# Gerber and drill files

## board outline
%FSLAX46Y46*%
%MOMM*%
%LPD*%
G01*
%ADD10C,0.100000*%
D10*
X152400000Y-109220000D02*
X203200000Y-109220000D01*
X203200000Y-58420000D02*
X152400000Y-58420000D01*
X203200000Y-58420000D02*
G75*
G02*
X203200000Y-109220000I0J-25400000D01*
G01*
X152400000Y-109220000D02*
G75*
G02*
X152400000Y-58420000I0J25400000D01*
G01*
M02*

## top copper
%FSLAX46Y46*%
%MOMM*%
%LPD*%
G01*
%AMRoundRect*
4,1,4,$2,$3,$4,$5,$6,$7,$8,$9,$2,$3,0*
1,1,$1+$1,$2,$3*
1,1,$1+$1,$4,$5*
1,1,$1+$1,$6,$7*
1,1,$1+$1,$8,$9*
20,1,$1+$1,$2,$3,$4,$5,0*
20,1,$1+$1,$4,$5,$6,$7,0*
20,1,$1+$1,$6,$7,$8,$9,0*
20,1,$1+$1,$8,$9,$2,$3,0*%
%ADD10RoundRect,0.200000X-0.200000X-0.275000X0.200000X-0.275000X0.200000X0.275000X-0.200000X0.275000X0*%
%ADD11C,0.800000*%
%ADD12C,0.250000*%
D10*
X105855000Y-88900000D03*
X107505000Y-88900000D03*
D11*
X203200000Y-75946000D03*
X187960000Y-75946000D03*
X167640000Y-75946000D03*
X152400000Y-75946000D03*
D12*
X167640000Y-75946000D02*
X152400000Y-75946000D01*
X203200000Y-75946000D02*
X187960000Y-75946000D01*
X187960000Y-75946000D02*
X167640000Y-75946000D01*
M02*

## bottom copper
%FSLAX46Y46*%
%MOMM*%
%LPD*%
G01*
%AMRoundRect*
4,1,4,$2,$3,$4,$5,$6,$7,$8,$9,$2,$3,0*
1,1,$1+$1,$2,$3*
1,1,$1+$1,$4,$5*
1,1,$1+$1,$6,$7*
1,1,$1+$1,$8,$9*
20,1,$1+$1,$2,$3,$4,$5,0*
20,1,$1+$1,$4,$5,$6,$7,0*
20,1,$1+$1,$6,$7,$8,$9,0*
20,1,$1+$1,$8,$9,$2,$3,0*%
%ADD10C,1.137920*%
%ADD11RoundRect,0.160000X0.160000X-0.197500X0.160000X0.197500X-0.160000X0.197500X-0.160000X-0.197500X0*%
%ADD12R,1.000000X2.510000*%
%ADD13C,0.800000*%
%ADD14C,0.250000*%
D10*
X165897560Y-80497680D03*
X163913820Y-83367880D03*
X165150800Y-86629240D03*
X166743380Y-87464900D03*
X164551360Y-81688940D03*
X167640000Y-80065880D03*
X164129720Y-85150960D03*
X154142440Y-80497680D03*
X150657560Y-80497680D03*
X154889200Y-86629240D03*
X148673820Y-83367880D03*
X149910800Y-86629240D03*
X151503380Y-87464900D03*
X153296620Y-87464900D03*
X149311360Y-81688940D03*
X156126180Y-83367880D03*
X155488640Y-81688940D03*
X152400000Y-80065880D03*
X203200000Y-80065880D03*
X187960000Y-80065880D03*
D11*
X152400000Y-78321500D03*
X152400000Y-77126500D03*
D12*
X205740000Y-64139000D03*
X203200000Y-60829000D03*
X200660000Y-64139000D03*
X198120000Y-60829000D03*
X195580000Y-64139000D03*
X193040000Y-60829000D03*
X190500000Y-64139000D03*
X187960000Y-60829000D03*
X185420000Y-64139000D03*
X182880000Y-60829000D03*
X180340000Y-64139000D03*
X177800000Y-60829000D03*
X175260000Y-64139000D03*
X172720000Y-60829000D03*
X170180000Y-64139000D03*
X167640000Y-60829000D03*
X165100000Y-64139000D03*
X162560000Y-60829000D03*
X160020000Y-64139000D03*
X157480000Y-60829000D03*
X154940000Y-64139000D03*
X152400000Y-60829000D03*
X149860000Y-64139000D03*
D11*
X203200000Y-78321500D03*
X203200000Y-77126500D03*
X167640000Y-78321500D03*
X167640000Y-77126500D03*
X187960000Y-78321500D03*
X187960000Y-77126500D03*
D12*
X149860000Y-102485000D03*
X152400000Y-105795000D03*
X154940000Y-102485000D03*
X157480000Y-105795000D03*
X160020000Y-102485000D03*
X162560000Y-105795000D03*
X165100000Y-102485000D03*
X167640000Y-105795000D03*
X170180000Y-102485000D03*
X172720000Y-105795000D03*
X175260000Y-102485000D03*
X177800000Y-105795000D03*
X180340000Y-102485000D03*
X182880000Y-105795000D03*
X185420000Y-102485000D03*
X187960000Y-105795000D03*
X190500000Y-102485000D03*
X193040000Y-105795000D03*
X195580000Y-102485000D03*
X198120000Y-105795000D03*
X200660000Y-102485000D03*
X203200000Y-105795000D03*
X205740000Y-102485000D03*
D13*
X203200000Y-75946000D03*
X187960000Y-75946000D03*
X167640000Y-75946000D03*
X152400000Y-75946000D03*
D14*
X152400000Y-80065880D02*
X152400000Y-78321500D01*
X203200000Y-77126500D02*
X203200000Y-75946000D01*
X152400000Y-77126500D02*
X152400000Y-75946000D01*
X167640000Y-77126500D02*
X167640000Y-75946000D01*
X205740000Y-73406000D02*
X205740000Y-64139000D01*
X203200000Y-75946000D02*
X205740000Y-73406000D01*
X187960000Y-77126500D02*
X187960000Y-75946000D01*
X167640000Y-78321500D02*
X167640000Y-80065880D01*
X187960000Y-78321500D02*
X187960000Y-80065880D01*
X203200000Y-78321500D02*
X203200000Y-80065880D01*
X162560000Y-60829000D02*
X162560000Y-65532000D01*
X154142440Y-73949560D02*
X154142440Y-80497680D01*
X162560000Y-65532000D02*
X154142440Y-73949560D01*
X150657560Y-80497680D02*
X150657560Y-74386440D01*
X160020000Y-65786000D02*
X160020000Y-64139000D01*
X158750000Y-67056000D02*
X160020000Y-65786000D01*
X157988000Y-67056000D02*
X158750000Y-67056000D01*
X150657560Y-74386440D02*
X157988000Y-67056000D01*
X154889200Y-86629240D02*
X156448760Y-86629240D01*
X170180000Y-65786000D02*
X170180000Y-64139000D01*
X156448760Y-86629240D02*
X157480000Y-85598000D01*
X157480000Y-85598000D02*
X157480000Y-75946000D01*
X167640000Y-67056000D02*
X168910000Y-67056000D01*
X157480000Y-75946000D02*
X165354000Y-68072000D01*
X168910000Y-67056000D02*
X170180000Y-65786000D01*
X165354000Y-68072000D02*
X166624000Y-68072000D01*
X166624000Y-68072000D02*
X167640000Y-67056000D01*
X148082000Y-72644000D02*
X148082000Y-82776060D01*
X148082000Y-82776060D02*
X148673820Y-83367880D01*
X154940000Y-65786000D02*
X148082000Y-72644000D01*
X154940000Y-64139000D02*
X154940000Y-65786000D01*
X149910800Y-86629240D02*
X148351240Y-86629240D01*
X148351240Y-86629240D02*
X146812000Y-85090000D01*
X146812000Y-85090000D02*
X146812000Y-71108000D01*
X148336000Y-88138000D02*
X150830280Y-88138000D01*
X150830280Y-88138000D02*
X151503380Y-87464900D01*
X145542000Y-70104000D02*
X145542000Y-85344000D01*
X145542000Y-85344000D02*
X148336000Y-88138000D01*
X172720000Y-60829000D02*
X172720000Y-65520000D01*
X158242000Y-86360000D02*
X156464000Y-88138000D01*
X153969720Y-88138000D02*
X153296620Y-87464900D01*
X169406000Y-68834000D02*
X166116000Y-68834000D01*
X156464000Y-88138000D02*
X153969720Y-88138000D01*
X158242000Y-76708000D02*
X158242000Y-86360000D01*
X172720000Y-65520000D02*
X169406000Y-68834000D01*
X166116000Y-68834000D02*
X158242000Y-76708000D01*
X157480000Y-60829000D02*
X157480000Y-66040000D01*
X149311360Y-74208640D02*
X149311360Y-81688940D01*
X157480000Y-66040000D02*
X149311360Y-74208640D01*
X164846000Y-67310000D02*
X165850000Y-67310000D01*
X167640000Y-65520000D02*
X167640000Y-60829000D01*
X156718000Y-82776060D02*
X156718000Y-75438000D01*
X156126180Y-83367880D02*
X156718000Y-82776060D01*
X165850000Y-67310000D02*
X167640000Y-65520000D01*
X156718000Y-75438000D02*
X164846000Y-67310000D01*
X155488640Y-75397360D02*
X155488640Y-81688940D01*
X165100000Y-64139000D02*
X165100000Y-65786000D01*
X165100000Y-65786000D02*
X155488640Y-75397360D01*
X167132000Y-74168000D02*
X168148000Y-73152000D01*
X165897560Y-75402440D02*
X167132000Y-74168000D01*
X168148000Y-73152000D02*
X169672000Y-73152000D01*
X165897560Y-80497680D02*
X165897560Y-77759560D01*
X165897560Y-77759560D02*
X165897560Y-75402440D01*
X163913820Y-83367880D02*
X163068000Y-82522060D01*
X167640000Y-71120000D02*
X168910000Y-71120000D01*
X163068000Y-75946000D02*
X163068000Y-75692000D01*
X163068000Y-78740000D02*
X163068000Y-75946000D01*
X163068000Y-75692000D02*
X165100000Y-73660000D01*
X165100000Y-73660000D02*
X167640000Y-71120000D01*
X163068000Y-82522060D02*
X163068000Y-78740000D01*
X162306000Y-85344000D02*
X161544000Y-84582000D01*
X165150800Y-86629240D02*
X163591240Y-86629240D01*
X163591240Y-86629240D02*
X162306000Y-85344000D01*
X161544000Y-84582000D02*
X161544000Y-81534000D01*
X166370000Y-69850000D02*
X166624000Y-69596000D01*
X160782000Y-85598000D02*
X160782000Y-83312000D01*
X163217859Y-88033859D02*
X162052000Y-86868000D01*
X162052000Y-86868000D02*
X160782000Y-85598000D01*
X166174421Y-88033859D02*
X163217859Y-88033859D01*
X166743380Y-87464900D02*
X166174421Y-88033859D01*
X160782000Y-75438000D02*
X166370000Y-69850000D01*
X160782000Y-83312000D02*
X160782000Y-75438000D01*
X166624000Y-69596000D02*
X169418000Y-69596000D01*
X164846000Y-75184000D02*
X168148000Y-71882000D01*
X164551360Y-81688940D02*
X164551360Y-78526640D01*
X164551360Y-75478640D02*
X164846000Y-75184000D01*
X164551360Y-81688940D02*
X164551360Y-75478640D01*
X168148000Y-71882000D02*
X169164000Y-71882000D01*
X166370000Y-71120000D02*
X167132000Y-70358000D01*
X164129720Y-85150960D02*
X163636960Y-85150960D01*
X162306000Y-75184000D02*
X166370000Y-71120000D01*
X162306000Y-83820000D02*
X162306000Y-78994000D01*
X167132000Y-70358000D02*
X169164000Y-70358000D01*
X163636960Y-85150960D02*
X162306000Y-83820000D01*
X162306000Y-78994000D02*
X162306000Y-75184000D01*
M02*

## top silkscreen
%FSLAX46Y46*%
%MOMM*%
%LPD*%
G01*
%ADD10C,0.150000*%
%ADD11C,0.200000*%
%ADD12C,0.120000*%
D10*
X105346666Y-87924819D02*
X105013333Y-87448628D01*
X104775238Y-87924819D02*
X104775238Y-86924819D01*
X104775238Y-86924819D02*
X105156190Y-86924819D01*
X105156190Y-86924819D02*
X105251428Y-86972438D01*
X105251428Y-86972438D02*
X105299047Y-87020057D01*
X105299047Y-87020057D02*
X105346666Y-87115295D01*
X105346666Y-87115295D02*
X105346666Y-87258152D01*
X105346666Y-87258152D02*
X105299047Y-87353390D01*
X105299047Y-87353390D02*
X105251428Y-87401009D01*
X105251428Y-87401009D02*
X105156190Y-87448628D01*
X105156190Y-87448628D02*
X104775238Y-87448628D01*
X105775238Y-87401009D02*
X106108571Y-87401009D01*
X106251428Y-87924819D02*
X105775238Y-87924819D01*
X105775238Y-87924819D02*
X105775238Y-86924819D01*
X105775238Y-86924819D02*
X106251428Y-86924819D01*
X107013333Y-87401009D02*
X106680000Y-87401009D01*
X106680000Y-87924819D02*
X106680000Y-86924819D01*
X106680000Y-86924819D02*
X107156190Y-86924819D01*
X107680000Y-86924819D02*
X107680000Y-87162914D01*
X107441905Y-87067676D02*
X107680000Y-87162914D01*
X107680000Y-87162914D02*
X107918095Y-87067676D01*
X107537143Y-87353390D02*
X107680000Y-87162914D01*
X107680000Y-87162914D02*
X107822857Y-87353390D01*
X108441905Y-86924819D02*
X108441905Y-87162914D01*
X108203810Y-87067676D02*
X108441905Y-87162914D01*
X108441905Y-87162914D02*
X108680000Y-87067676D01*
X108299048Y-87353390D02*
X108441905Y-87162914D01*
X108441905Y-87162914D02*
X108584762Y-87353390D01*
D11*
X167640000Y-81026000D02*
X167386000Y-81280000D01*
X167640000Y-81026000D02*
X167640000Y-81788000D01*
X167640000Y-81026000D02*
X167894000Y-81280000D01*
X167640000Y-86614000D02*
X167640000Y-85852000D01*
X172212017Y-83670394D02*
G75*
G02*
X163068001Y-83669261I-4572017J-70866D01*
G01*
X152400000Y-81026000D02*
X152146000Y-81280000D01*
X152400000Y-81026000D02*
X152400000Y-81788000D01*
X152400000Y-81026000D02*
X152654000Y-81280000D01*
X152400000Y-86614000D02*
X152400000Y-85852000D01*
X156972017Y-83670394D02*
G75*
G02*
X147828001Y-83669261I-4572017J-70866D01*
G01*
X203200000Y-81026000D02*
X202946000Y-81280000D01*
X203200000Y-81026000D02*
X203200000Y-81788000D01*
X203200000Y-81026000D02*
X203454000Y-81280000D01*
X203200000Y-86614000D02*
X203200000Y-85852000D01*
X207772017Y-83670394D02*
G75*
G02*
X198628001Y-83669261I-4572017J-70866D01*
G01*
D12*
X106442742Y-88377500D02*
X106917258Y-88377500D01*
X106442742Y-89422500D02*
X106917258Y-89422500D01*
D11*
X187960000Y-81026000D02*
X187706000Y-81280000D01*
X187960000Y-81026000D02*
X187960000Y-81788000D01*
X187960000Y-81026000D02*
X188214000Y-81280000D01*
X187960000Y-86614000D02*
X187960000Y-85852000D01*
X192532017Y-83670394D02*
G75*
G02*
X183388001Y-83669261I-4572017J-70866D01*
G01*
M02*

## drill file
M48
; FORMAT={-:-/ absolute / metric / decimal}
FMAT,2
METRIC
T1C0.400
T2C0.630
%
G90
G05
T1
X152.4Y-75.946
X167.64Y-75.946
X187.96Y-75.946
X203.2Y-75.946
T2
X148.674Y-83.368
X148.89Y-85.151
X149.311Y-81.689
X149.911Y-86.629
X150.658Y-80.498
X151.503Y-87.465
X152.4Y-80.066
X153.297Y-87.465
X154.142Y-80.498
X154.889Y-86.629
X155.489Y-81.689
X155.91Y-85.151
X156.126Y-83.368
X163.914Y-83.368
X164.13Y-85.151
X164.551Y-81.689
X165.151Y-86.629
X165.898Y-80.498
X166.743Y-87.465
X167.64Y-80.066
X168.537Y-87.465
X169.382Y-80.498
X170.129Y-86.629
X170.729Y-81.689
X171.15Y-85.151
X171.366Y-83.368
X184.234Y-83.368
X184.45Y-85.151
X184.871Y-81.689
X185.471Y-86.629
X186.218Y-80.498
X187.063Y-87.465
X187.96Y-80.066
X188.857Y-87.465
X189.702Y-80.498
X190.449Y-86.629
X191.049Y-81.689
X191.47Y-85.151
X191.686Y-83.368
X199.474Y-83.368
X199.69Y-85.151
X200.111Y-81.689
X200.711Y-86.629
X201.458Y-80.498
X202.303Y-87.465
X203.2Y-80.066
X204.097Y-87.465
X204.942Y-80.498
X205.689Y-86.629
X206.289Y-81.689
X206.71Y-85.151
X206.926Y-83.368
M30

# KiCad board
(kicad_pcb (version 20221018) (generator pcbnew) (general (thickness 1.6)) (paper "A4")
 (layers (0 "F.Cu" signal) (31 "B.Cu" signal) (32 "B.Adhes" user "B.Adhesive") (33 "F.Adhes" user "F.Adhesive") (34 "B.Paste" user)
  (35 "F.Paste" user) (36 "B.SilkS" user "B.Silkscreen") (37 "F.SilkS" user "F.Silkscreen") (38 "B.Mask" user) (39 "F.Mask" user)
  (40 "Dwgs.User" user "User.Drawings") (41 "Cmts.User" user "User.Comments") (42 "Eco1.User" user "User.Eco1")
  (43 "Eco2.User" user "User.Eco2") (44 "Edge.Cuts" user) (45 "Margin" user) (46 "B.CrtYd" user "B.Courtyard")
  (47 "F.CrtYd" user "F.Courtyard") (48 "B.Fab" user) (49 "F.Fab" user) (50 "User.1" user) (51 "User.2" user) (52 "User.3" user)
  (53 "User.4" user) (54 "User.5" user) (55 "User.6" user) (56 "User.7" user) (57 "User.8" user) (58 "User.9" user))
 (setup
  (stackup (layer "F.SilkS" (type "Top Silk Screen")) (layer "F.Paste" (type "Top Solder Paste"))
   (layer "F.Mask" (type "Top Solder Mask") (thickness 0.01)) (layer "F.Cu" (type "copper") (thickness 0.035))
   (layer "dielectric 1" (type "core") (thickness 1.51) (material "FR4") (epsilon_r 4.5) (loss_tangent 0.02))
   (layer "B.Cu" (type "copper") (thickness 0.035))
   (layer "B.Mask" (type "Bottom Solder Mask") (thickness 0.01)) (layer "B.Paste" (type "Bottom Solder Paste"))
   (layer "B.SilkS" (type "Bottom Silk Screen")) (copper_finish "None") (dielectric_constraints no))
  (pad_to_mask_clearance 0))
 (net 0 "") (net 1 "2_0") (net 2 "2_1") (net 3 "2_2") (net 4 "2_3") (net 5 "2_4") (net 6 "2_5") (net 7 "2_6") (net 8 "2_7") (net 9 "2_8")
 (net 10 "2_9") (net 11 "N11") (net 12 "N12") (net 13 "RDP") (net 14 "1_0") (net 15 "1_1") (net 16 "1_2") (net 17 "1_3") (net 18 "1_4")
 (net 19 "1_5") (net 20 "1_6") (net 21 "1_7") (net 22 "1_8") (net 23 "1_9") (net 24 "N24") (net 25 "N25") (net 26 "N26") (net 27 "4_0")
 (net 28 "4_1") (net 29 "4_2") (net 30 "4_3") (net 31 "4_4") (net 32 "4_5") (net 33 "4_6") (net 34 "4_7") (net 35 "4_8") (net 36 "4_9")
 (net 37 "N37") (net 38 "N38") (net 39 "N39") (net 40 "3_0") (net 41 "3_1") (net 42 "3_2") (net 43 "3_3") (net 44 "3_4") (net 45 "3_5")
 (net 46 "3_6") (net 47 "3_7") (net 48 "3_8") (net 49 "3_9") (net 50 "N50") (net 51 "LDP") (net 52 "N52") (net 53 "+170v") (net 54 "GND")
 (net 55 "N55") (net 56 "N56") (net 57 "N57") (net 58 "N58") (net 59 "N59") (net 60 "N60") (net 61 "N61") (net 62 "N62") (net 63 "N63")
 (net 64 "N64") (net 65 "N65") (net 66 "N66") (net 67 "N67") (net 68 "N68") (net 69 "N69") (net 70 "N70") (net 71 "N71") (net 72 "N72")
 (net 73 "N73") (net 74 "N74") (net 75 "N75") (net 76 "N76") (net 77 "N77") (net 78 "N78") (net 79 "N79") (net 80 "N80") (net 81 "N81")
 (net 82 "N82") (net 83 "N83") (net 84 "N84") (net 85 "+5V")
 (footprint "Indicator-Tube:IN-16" (layer "F.Cu") (at 167.64 83.82)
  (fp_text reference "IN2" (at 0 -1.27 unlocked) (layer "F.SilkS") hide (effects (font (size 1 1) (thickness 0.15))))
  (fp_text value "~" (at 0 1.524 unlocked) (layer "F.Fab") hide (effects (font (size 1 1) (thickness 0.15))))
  (fp_line (start 0 -2.794) (end -0.254 -2.54) (stroke (width 0.2) (type solid)) (layer "F.SilkS"))
  (fp_line (start 0 -2.794) (end 0 -2.032) (stroke (width 0.2) (type solid)) (layer "F.SilkS"))
  (fp_line (start 0 -2.794) (end 0.254 -2.54) (stroke (width 0.2) (type solid)) (layer "F.SilkS"))
  (fp_line (start 0 2.794) (end 0 2.032) (stroke (width 0.2) (type solid)) (layer "F.SilkS"))
  (fp_arc (start 4.572017 -0.149606) (mid -0.000567 4.493826) (end -4.571999 -0.150739) (stroke (width 0.2) (type solid)) (layer "F.SilkS"))
  (pad "0" thru_hole circle (at 1.74244 -3.32232 180) (size 1.13792 1.13792) (drill 0.62992) (layers "*.Cu" "*.Mask") (remove_unused_layers)
   (zone_layer_connections) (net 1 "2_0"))
  (pad "1" thru_hole circle (at -1.74244 -3.32232 180) (size 1.13792 1.13792) (drill 0.62992) (layers "*.Cu" "*.Mask")
   (remove_unused_layers) (zone_layer_connections) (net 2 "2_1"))
  (pad "2" thru_hole circle (at 2.4892 2.80924 180) (size 1.13792 1.13792) (drill 0.62992) (layers "*.Cu" "*.Mask") (remove_unused_layers)
   (zone_layer_connections) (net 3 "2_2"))
  (pad "3" thru_hole circle (at -3.72618 -0.45212 180) (size 1.13792 1.13792) (drill 0.62992) (layers "*.Cu" "*.Mask")
   (remove_unused_layers) (zone_layer_connections) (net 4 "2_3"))
  (pad "4" thru_hole circle (at -2.4892 2.80924 180) (size 1.13792 1.13792) (drill 0.62992) (layers "*.Cu" "*.Mask") (remove_unused_layers)
   (zone_layer_connections) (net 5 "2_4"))
  (pad "5" thru_hole circle (at -0.89662 3.6449 180) (size 1.13792 1.13792) (drill 0.62992) (layers "*.Cu" "*.Mask") (remove_unused_layers)
   (zone_layer_connections) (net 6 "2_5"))
  (pad "6" thru_hole circle (at 0.89662 3.6449 180) (size 1.13792 1.13792) (drill 0.62992) (layers "*.Cu" "*.Mask") (remove_unused_layers)
   (zone_layer_connections) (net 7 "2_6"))
  (pad "7" thru_hole circle (at -3.08864 -2.13106 180) (size 1.13792 1.13792) (drill 0.62992) (layers "*.Cu" "*.Mask")
   (remove_unused_layers) (zone_layer_connections) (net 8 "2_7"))
  (pad "8" thru_hole circle (at 3.72618 -0.45212 180) (size 1.13792 1.13792) (drill 0.62992) (layers "*.Cu" "*.Mask") (remove_unused_layers)
   (zone_layer_connections) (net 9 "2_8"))
  (pad "9" thru_hole circle (at 3.08864 -2.13106 180) (size 1.13792 1.13792) (drill 0.62992) (layers "*.Cu" "*.Mask") (remove_unused_layers)
   (zone_layer_connections) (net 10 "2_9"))
  (pad "A" thru_hole circle (at 0 -3.75412 180) (size 1.13792 1.13792) (drill 0.62992) (layers "*.Cu" "*.Mask") (remove_unused_layers)
   (zone_layer_connections) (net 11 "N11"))
  (pad "LHDP" thru_hole circle (at 3.51028 1.33096 180) (size 1.13792 1.13792) (drill 0.62992) (layers "*.Cu" "*.Mask")
   (remove_unused_layers) (zone_layer_connections) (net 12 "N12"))
  (pad "RHDP" thru_hole circle (at -3.51028 1.33096 180) (size 1.13792 1.13792) (drill 0.62992) (layers "*.Cu" "*.Mask")
   (remove_unused_layers) (zone_layer_connections) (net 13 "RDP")))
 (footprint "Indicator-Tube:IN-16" (layer "F.Cu") (at 152.4 83.82)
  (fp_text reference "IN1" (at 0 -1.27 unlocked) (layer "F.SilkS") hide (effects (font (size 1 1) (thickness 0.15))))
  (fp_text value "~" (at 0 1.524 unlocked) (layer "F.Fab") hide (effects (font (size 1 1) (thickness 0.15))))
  (fp_line (start 0 -2.794) (end -0.254 -2.54) (stroke (width 0.2) (type solid)) (layer "F.SilkS"))
  (fp_line (start 0 -2.794) (end 0 -2.032) (stroke (width 0.2) (type solid)) (layer "F.SilkS"))
  (fp_line (start 0 -2.794) (end 0.254 -2.54) (stroke (width 0.2) (type solid)) (layer "F.SilkS"))
  (fp_line (start 0 2.794) (end 0 2.032) (stroke (width 0.2) (type solid)) (layer "F.SilkS"))
  (fp_arc (start 4.572017 -0.149606) (mid -0.000567 4.493826) (end -4.571999 -0.150739) (stroke (width 0.2) (type solid)) (layer "F.SilkS"))
  (pad "0" thru_hole circle (at 1.74244 -3.32232 180) (size 1.13792 1.13792) (drill 0.62992) (layers "*.Cu" "*.Mask") (remove_unused_layers)
   (zone_layer_connections) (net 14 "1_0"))
  (pad "1" thru_hole circle (at -1.74244 -3.32232 180) (size 1.13792 1.13792) (drill 0.62992) (layers "*.Cu" "*.Mask")
   (remove_unused_layers) (zone_layer_connections) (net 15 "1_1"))
  (pad "2" thru_hole circle (at 2.4892 2.80924 180) (size 1.13792 1.13792) (drill 0.62992) (layers "*.Cu" "*.Mask") (remove_unused_layers)
   (zone_layer_connections) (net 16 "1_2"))
  (pad "3" thru_hole circle (at -3.72618 -0.45212 180) (size 1.13792 1.13792) (drill 0.62992) (layers "*.Cu" "*.Mask")
   (remove_unused_layers) (zone_layer_connections) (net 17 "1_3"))
  (pad "4" thru_hole circle (at -2.4892 2.80924 180) (size 1.13792 1.13792) (drill 0.62992) (layers "*.Cu" "*.Mask") (remove_unused_layers)
   (zone_layer_connections) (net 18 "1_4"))
  (pad "5" thru_hole circle (at -0.89662 3.6449 180) (size 1.13792 1.13792) (drill 0.62992) (layers "*.Cu" "*.Mask") (remove_unused_layers)
   (zone_layer_connections) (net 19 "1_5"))
  (pad "6" thru_hole circle (at 0.89662 3.6449 180) (size 1.13792 1.13792) (drill 0.62992) (layers "*.Cu" "*.Mask") (remove_unused_layers)
   (zone_layer_connections) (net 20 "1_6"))
  (pad "7" thru_hole circle (at -3.08864 -2.13106 180) (size 1.13792 1.13792) (drill 0.62992) (layers "*.Cu" "*.Mask")
   (remove_unused_layers) (zone_layer_connections) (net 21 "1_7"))
  (pad "8" thru_hole circle (at 3.72618 -0.45212 180) (size 1.13792 1.13792) (drill 0.62992) (layers "*.Cu" "*.Mask") (remove_unused_layers)
   (zone_layer_connections) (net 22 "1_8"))
  (pad "9" thru_hole circle (at 3.08864 -2.13106 180) (size 1.13792 1.13792) (drill 0.62992) (layers "*.Cu" "*.Mask") (remove_unused_layers)
   (zone_layer_connections) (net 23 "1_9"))
  (pad "A" thru_hole circle (at 0 -3.75412 180) (size 1.13792 1.13792) (drill 0.62992) (layers "*.Cu" "*.Mask") (remove_unused_layers)
   (zone_layer_connections) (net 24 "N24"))
  (pad "LHDP" thru_hole circle (at 3.51028 1.33096 180) (size 1.13792 1.13792) (drill 0.62992) (layers "*.Cu" "*.Mask")
   (remove_unused_layers) (zone_layer_connections) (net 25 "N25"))
  (pad "RHDP" thru_hole circle (at -3.51028 1.33096 180) (size 1.13792 1.13792) (drill 0.62992) (layers "*.Cu" "*.Mask")
   (remove_unused_layers) (zone_layer_connections) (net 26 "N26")))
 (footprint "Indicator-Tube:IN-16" (layer "F.Cu") (at 203.2 83.82)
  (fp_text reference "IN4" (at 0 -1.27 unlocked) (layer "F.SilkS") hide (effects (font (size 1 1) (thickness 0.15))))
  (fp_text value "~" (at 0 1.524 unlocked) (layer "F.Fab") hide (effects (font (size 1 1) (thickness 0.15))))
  (fp_line (start 0 -2.794) (end -0.254 -2.54) (stroke (width 0.2) (type solid)) (layer "F.SilkS"))
  (fp_line (start 0 -2.794) (end 0 -2.032) (stroke (width 0.2) (type solid)) (layer "F.SilkS"))
  (fp_line (start 0 -2.794) (end 0.254 -2.54) (stroke (width 0.2) (type solid)) (layer "F.SilkS"))
  (fp_line (start 0 2.794) (end 0 2.032) (stroke (width 0.2) (type solid)) (layer "F.SilkS"))
  (fp_arc (start 4.572017 -0.149606) (mid -0.000567 4.493826) (end -4.571999 -0.150739) (stroke (width 0.2) (type solid)) (layer "F.SilkS"))
  (pad "0" thru_hole circle (at 1.74244 -3.32232 180) (size 1.13792 1.13792) (drill 0.62992) (layers "*.Cu" "*.Mask") (remove_unused_layers)
   (zone_layer_connections) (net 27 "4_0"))
  (pad "1" thru_hole circle (at -1.74244 -3.32232 180) (size 1.13792 1.13792) (drill 0.62992) (layers "*.Cu" "*.Mask")
   (remove_unused_layers) (zone_layer_connections) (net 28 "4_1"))
  (pad "2" thru_hole circle (at 2.4892 2.80924 180) (size 1.13792 1.13792) (drill 0.62992) (layers "*.Cu" "*.Mask") (remove_unused_layers)
   (zone_layer_connections) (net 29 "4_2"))
  (pad "3" thru_hole circle (at -3.72618 -0.45212 180) (size 1.13792 1.13792) (drill 0.62992) (layers "*.Cu" "*.Mask")
   (remove_unused_layers) (zone_layer_connections) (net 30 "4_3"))
  (pad "4" thru_hole circle (at -2.4892 2.80924 180) (size 1.13792 1.13792) (drill 0.62992) (layers "*.Cu" "*.Mask") (remove_unused_layers)
   (zone_layer_connections) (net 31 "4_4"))
  (pad "5" thru_hole circle (at -0.89662 3.6449 180) (size 1.13792 1.13792) (drill 0.62992) (layers "*.Cu" "*.Mask") (remove_unused_layers)
   (zone_layer_connections) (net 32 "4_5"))
  (pad "6" thru_hole circle (at 0.89662 3.6449 180) (size 1.13792 1.13792) (drill 0.62992) (layers "*.Cu" "*.Mask") (remove_unused_layers)
   (zone_layer_connections) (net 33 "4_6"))
  (pad "7" thru_hole circle (at -3.08864 -2.13106 180) (size 1.13792 1.13792) (drill 0.62992) (layers "*.Cu" "*.Mask")
   (remove_unused_layers) (zone_layer_connections) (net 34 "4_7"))
  (pad "8" thru_hole circle (at 3.72618 -0.45212 180) (size 1.13792 1.13792) (drill 0.62992) (layers "*.Cu" "*.Mask") (remove_unused_layers)
   (zone_layer_connections) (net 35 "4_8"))
  (pad "9" thru_hole circle (at 3.08864 -2.13106 180) (size 1.13792 1.13792) (drill 0.62992) (layers "*.Cu" "*.Mask") (remove_unused_layers)
   (zone_layer_connections) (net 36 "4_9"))
  (pad "A" thru_hole circle (at 0 -3.75412 180) (size 1.13792 1.13792) (drill 0.62992) (layers "*.Cu" "*.Mask") (remove_unused_layers)
   (zone_layer_connections) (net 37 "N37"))
  (pad "LHDP" thru_hole circle (at 3.51028 1.33096 180) (size 1.13792 1.13792) (drill 0.62992) (layers "*.Cu" "*.Mask")
   (remove_unused_layers) (zone_layer_connections) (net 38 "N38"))
  (pad "RHDP" thru_hole circle (at -3.51028 1.33096 180) (size 1.13792 1.13792) (drill 0.62992) (layers "*.Cu" "*.Mask")
   (remove_unused_layers) (zone_layer_connections) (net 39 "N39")))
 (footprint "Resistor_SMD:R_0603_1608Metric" (layer "F.Cu") (at 106.68 88.9)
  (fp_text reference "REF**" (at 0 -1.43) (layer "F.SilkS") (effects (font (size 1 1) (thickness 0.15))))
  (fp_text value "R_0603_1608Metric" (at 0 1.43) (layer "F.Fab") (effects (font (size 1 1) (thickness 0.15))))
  (fp_line (start -0.237258 -0.5225) (end 0.237258 -0.5225) (stroke (width 0.12) (type solid)) (layer "F.SilkS"))
  (fp_line (start -0.237258 0.5225) (end 0.237258 0.5225) (stroke (width 0.12) (type solid)) (layer "F.SilkS"))
  (pad "1" smd roundrect (at -0.825 0) (size 0.8 0.95) (layers "F.Cu" "F.Paste" "F.Mask") (roundrect_rratio 0.25))
  (pad "2" smd roundrect (at 0.825 0) (size 0.8 0.95) (layers "F.Cu" "F.Paste" "F.Mask") (roundrect_rratio 0.25)))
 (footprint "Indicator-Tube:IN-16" (layer "F.Cu") (at 187.96 83.82)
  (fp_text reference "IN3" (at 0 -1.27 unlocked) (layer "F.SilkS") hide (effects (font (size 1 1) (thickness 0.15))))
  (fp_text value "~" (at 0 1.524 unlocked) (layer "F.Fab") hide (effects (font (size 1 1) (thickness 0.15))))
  (fp_line (start 0 -2.794) (end -0.254 -2.54) (stroke (width 0.2) (type solid)) (layer "F.SilkS"))
  (fp_line (start 0 -2.794) (end 0 -2.032) (stroke (width 0.2) (type solid)) (layer "F.SilkS"))
  (fp_line (start 0 -2.794) (end 0.254 -2.54) (stroke (width 0.2) (type solid)) (layer "F.SilkS"))
  (fp_line (start 0 2.794) (end 0 2.032) (stroke (width 0.2) (type solid)) (layer "F.SilkS"))
  (fp_arc (start 4.572017 -0.149606) (mid -0.000567 4.493826) (end -4.571999 -0.150739) (stroke (width 0.2) (type solid)) (layer "F.SilkS"))
  (pad "0" thru_hole circle (at 1.74244 -3.32232 180) (size 1.13792 1.13792) (drill 0.62992) (layers "*.Cu" "*.Mask") (remove_unused_layers)
   (zone_layer_connections) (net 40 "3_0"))
  (pad "1" thru_hole circle (at -1.74244 -3.32232 180) (size 1.13792 1.13792) (drill 0.62992) (layers "*.Cu" "*.Mask")
   (remove_unused_layers) (zone_layer_connections) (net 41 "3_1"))
  (pad "2" thru_hole circle (at 2.4892 2.80924 180) (size 1.13792 1.13792) (drill 0.62992) (layers "*.Cu" "*.Mask") (remove_unused_layers)
   (zone_layer_connections) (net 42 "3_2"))
  (pad "3" thru_hole circle (at -3.72618 -0.45212 180) (size 1.13792 1.13792) (drill 0.62992) (layers "*.Cu" "*.Mask")
   (remove_unused_layers) (zone_layer_connections) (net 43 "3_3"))
  (pad "4" thru_hole circle (at -2.4892 2.80924 180) (size 1.13792 1.13792) (drill 0.62992) (layers "*.Cu" "*.Mask") (remove_unused_layers)
   (zone_layer_connections) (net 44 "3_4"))
  (pad "5" thru_hole circle (at -0.89662 3.6449 180) (size 1.13792 1.13792) (drill 0.62992) (layers "*.Cu" "*.Mask") (remove_unused_layers)
   (zone_layer_connections) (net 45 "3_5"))
  (pad "6" thru_hole circle (at 0.89662 3.6449 180) (size 1.13792 1.13792) (drill 0.62992) (layers "*.Cu" "*.Mask") (remove_unused_layers)
   (zone_layer_connections) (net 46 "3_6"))
  (pad "7" thru_hole circle (at -3.08864 -2.13106 180) (size 1.13792 1.13792) (drill 0.62992) (layers "*.Cu" "*.Mask")
   (remove_unused_layers) (zone_layer_connections) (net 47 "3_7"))
  (pad "8" thru_hole circle (at 3.72618 -0.45212 180) (size 1.13792 1.13792) (drill 0.62992) (layers "*.Cu" "*.Mask") (remove_unused_layers)
   (zone_layer_connections) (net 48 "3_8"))
  (pad "9" thru_hole circle (at 3.08864 -2.13106 180) (size 1.13792 1.13792) (drill 0.62992) (layers "*.Cu" "*.Mask") (remove_unused_layers)
   (zone_layer_connections) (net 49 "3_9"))
  (pad "A" thru_hole circle (at 0 -3.75412 180) (size 1.13792 1.13792) (drill 0.62992) (layers "*.Cu" "*.Mask") (remove_unused_layers)
   (zone_layer_connections) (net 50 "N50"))
  (pad "LHDP" thru_hole circle (at 3.51028 1.33096 180) (size 1.13792 1.13792) (drill 0.62992) (layers "*.Cu" "*.Mask")
   (remove_unused_layers) (zone_layer_connections) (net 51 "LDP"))
  (pad "RHDP" thru_hole circle (at -3.51028 1.33096 180) (size 1.13792 1.13792) (drill 0.62992) (layers "*.Cu" "*.Mask")
   (remove_unused_layers) (zone_layer_connections) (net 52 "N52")))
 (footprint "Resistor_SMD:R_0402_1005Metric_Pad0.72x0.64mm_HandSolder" (layer "B.Cu") (at 152.4 77.724 90)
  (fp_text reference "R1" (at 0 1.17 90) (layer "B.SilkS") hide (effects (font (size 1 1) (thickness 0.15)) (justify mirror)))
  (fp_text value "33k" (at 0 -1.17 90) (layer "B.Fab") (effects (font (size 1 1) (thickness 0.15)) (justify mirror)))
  (pad "1" smd roundrect (at -0.5975 0 90) (size 0.715 0.64) (layers "B.Cu" "B.Paste" "B.Mask") (roundrect_rratio 0.25) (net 24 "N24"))
  (pad "2" smd roundrect (at 0.5975 0 90) (size 0.715 0.64) (layers "B.Cu" "B.Paste" "B.Mask") (roundrect_rratio 0.25) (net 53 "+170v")))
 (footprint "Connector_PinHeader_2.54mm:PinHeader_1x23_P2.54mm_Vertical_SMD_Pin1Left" (layer "B.Cu") (at 177.8 62.484 90)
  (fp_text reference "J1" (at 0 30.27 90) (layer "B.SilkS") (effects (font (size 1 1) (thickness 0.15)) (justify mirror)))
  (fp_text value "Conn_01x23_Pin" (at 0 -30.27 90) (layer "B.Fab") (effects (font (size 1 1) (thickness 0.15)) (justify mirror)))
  (pad "1" smd rect (at -1.655 27.94 90) (size 2.51 1) (layers "B.Cu" "B.Paste" "B.Mask") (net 53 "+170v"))
  (pad "2" smd rect (at 1.655 25.4 90) (size 2.51 1) (layers "B.Cu" "B.Paste" "B.Mask") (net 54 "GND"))
  (pad "3" smd rect (at -1.655 22.86 90) (size 2.51 1) (layers "B.Cu" "B.Paste" "B.Mask") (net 13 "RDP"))
  (pad "4" smd rect (at 1.655 20.32 90) (size 2.51 1) (layers "B.Cu" "B.Paste" "B.Mask") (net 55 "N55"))
  (pad "5" smd rect (at -1.655 17.78 90) (size 2.51 1) (layers "B.Cu" "B.Paste" "B.Mask") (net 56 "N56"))
  (pad "6" smd rect (at 1.655 15.24 90) (size 2.51 1) (layers "B.Cu" "B.Paste" "B.Mask") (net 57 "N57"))
  (pad "7" smd rect (at -1.655 12.7 90) (size 2.51 1) (layers "B.Cu" "B.Paste" "B.Mask") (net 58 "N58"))
  (pad "8" smd rect (at 1.655 10.16 90) (size 2.51 1) (layers "B.Cu" "B.Paste" "B.Mask") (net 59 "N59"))
  (pad "9" smd rect (at -1.655 7.62 90) (size 2.51 1) (layers "B.Cu" "B.Paste" "B.Mask") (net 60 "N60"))
  (pad "10" smd rect (at 1.655 5.08 90) (size 2.51 1) (layers "B.Cu" "B.Paste" "B.Mask") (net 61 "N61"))
  (pad "11" smd rect (at -1.655 2.54 90) (size 2.51 1) (layers "B.Cu" "B.Paste" "B.Mask") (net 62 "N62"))
  (pad "12" smd rect (at 1.655 0 90) (size 2.51 1) (layers "B.Cu" "B.Paste" "B.Mask") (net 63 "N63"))
  (pad "13" smd rect (at -1.655 -2.54 90) (size 2.51 1) (layers "B.Cu" "B.Paste" "B.Mask") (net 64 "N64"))
  (pad "14" smd rect (at 1.655 -5.08 90) (size 2.51 1) (layers "B.Cu" "B.Paste" "B.Mask") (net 20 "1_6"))
  (pad "15" smd rect (at -1.655 -7.62 90) (size 2.51 1) (layers "B.Cu" "B.Paste" "B.Mask") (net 16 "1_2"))
  (pad "16" smd rect (at 1.655 -10.16 90) (size 2.51 1) (layers "B.Cu" "B.Paste" "B.Mask") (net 22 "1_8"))
  (pad "17" smd rect (at -1.655 -12.7 90) (size 2.51 1) (layers "B.Cu" "B.Paste" "B.Mask") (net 23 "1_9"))
  (pad "18" smd rect (at 1.655 -15.24 90) (size 2.51 1) (layers "B.Cu" "B.Paste" "B.Mask") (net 14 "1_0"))
  (pad "19" smd rect (at -1.655 -17.78 90) (size 2.51 1) (layers "B.Cu" "B.Paste" "B.Mask") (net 15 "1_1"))
  (pad "20" smd rect (at 1.655 -20.32 90) (size 2.51 1) (layers "B.Cu" "B.Paste" "B.Mask") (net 21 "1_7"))
  (pad "21" smd rect (at -1.655 -22.86 90) (size 2.51 1) (layers "B.Cu" "B.Paste" "B.Mask") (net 17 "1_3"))
  (pad "22" smd rect (at 1.655 -25.4 90) (size 2.51 1) (layers "B.Cu" "B.Paste" "B.Mask") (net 18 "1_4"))
  (pad "23" smd rect (at -1.655 -27.94 90) (size 2.51 1) (layers "B.Cu" "B.Paste" "B.Mask") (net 19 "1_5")))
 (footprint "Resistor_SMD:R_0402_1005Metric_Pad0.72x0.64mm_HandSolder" (layer "B.Cu") (at 203.2 77.724 90)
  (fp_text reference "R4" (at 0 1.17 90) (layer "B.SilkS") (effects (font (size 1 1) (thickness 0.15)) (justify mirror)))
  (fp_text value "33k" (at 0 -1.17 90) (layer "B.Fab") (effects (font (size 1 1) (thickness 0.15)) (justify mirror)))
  (pad "1" smd roundrect (at -0.5975 0 90) (size 0.715 0.64) (layers "B.Cu" "B.Paste" "B.Mask") (roundrect_rratio 0.25) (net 37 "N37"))
  (pad "2" smd roundrect (at 0.5975 0 90) (size 0.715 0.64) (layers "B.Cu" "B.Paste" "B.Mask") (roundrect_rratio 0.25) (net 53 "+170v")))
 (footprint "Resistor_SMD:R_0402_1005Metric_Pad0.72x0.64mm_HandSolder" (layer "B.Cu") (at 167.64 77.724 90)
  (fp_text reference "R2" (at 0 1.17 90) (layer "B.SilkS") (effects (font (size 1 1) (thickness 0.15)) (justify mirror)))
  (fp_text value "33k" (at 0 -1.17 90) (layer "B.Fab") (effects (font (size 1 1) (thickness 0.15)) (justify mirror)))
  (pad "1" smd roundrect (at -0.5975 0 90) (size 0.715 0.64) (layers "B.Cu" "B.Paste" "B.Mask") (roundrect_rratio 0.25) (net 11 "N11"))
  (pad "2" smd roundrect (at 0.5975 0 90) (size 0.715 0.64) (layers "B.Cu" "B.Paste" "B.Mask") (roundrect_rratio 0.25) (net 53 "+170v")))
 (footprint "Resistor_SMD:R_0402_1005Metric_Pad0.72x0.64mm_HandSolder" (layer "B.Cu") (at 187.96 77.724 90)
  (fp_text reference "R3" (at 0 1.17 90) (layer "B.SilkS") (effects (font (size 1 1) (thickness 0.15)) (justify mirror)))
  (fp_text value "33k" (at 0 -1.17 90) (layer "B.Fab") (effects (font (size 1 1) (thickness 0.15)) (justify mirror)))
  (pad "1" smd roundrect (at -0.5975 0 90) (size 0.715 0.64) (layers "B.Cu" "B.Paste" "B.Mask") (roundrect_rratio 0.25) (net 50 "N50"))
  (pad "2" smd roundrect (at 0.5975 0 90) (size 0.715 0.64) (layers "B.Cu" "B.Paste" "B.Mask") (roundrect_rratio 0.25) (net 53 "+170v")))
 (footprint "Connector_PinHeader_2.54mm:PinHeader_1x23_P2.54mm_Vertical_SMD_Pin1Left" (layer "B.Cu") (at 177.8 104.14 -90)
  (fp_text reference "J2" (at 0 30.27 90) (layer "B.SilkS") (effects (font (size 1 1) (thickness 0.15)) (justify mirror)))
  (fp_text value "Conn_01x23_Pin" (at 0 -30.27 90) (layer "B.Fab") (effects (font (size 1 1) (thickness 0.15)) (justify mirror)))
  (pad "1" smd rect (at -1.655 27.94 270) (size 2.51 1) (layers "B.Cu" "B.Paste" "B.Mask") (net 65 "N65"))
  (pad "2" smd rect (at 1.655 25.4 270) (size 2.51 1) (layers "B.Cu" "B.Paste" "B.Mask") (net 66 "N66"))
  (pad "3" smd rect (at -1.655 22.86 270) (size 2.51 1) (layers "B.Cu" "B.Paste" "B.Mask") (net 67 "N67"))
  (pad "4" smd rect (at 1.655 20.32 270) (size 2.51 1) (layers "B.Cu" "B.Paste" "B.Mask") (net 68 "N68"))
  (pad "5" smd rect (at -1.655 17.78 270) (size 2.51 1) (layers "B.Cu" "B.Paste" "B.Mask") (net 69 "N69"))
  (pad "6" smd rect (at 1.655 15.24 270) (size 2.51 1) (layers "B.Cu" "B.Paste" "B.Mask") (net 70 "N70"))
  (pad "7" smd rect (at -1.655 12.7 270) (size 2.51 1) (layers "B.Cu" "B.Paste" "B.Mask") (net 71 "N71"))
  (pad "8" smd rect (at 1.655 10.16 270) (size 2.51 1) (layers "B.Cu" "B.Paste" "B.Mask") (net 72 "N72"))
  (pad "9" smd rect (at -1.655 7.62 270) (size 2.51 1) (layers "B.Cu" "B.Paste" "B.Mask") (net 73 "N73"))
  (pad "10" smd rect (at 1.655 5.08 270) (size 2.51 1) (layers "B.Cu" "B.Paste" "B.Mask") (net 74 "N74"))
  (pad "11" smd rect (at -1.655 2.54 270) (size 2.51 1) (layers "B.Cu" "B.Paste" "B.Mask") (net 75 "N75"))
  (pad "12" smd rect (at 1.655 0 270) (size 2.51 1) (layers "B.Cu" "B.Paste" "B.Mask") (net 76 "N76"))
  (pad "13" smd rect (at -1.655 -2.54 270) (size 2.51 1) (layers "B.Cu" "B.Paste" "B.Mask") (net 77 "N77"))
  (pad "14" smd rect (at 1.655 -5.08 270) (size 2.51 1) (layers "B.Cu" "B.Paste" "B.Mask") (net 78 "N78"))
  (pad "15" smd rect (at -1.655 -7.62 270) (size 2.51 1) (layers "B.Cu" "B.Paste" "B.Mask") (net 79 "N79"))
  (pad "16" smd rect (at 1.655 -10.16 270) (size 2.51 1) (layers "B.Cu" "B.Paste" "B.Mask") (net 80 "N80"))
  (pad "17" smd rect (at -1.655 -12.7 270) (size 2.51 1) (layers "B.Cu" "B.Paste" "B.Mask") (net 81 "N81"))
  (pad "18" smd rect (at 1.655 -15.24 270) (size 2.51 1) (layers "B.Cu" "B.Paste" "B.Mask") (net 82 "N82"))
  (pad "19" smd rect (at -1.655 -17.78 270) (size 2.51 1) (layers "B.Cu" "B.Paste" "B.Mask") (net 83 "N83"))
  (pad "20" smd rect (at 1.655 -20.32 270) (size 2.51 1) (layers "B.Cu" "B.Paste" "B.Mask") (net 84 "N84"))
  (pad "21" smd rect (at -1.655 -22.86 270) (size 2.51 1) (layers "B.Cu" "B.Paste" "B.Mask") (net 51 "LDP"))
  (pad "22" smd rect (at 1.655 -25.4 270) (size 2.51 1) (layers "B.Cu" "B.Paste" "B.Mask") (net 54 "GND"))
  (pad "23" smd rect (at -1.655 -27.94 270) (size 2.51 1) (layers "B.Cu" "B.Paste" "B.Mask") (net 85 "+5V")))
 (gr_line (start 152.4 109.22) (end 203.2 109.22) (stroke (width 0.1) (type default)) (layer "Edge.Cuts"))
 (gr_line (start 203.2 58.42) (end 152.4 58.42) (stroke (width 0.1) (type default)) (layer "Edge.Cuts"))
 (gr_arc (start 203.2 58.42) (mid 228.6 83.82) (end 203.2 109.22) (stroke (width 0.1) (type default)) (layer "Edge.Cuts"))
 (gr_arc (start 152.4 109.22) (mid 127 83.82) (end 152.4 58.42) (stroke (width 0.1) (type default)) (layer "Edge.Cuts"))
 (segment (start 152.4 80.06588) (end 152.4 78.3215) (width 0.25) (layer "B.Cu") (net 24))
 (segment (start 167.64 75.946) (end 152.4 75.946) (width 0.25) (layer "F.Cu") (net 53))
 (segment (start 203.2 75.946) (end 187.96 75.946) (width 0.25) (layer "F.Cu") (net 53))
 (segment (start 187.96 75.946) (end 167.64 75.946) (width 0.25) (layer "F.Cu") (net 53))
 (via (at 203.2 75.946) (size 0.8) (drill 0.4) (layers "F.Cu" "B.Cu") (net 53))
 (via (at 187.96 75.946) (size 0.8) (drill 0.4) (layers "F.Cu" "B.Cu") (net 53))
 (via (at 167.64 75.946) (size 0.8) (drill 0.4) (layers "F.Cu" "B.Cu") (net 53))
 (via (at 152.4 75.946) (size 0.8) (drill 0.4) (layers "F.Cu" "B.Cu") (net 53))
 (segment (start 203.2 77.1265) (end 203.2 75.946) (width 0.25) (layer "B.Cu") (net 53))
 (segment (start 152.4 77.1265) (end 152.4 75.946) (width 0.25) (layer "B.Cu") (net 53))
 (segment (start 167.64 77.1265) (end 167.64 75.946) (width 0.25) (layer "B.Cu") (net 53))
 (segment (start 205.74 73.406) (end 205.74 64.139) (width 0.25) (layer "B.Cu") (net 53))
 (segment (start 203.2 75.946) (end 205.74 73.406) (width 0.25) (layer "B.Cu") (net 53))
 (segment (start 187.96 77.1265) (end 187.96 75.946) (width 0.25) (layer "B.Cu") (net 53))
 (segment (start 167.64 78.3215) (end 167.64 80.06588) (width 0.25) (layer "B.Cu") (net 11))
 (segment (start 187.96 78.3215) (end 187.96 80.06588) (width 0.25) (layer "B.Cu") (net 50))
 (segment (start 203.2 78.3215) (end 203.2 80.06588) (width 0.25) (layer "B.Cu") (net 37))
 (segment (start 162.56 60.829) (end 162.56 65.532) (width 0.25) (layer "B.Cu") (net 14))
 (segment (start 154.14244 73.94956) (end 154.14244 80.49768) (width 0.25) (layer "B.Cu") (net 14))
 (segment (start 162.56 65.532) (end 154.14244 73.94956) (width 0.25) (layer "B.Cu") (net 14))
 (segment (start 150.65756 80.49768) (end 150.65756 74.38644) (width 0.25) (layer "B.Cu") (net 15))
 (segment (start 160.02 65.786) (end 160.02 64.139) (width 0.25) (layer "B.Cu") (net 15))
 (segment (start 158.75 67.056) (end 160.02 65.786) (width 0.25) (layer "B.Cu") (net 15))
 (segment (start 157.988 67.056) (end 158.75 67.056) (width 0.25) (layer "B.Cu") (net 15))
 (segment (start 150.65756 74.38644) (end 157.988 67.056) (width 0.25) (layer "B.Cu") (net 15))
 (segment (start 154.8892 86.62924) (end 156.44876 86.62924) (width 0.25) (layer "B.Cu") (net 16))
 (segment (start 170.18 65.786) (end 170.18 64.139) (width 0.25) (layer "B.Cu") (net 16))
 (segment (start 156.44876 86.62924) (end 157.48 85.598) (width 0.25) (layer "B.Cu") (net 16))
 (segment (start 157.48 85.598) (end 157.48 75.946) (width 0.25) (layer "B.Cu") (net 16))
 (segment (start 167.64 67.056) (end 168.91 67.056) (width 0.25) (layer "B.Cu") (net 16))
 (segment (start 157.48 75.946) (end 165.354 68.072) (width 0.25) (layer "B.Cu") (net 16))
 (segment (start 168.91 67.056) (end 170.18 65.786) (width 0.25) (layer "B.Cu") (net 16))
 (segment (start 165.354 68.072) (end 166.624 68.072) (width 0.25) (layer "B.Cu") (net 16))
 (segment (start 166.624 68.072) (end 167.64 67.056) (width 0.25) (layer "B.Cu") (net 16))
 (segment (start 148.082 72.644) (end 148.082 82.77606) (width 0.25) (layer "B.Cu") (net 17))
 (segment (start 148.082 82.77606) (end 148.67382 83.36788) (width 0.25) (layer "B.Cu") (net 17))
 (segment (start 154.94 65.786) (end 148.082 72.644) (width 0.25) (layer "B.Cu") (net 17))
 (segment (start 154.94 64.139) (end 154.94 65.786) (width 0.25) (layer "B.Cu") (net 17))
 (segment (start 149.9108 86.62924) (end 148.35124 86.62924) (width 0.25) (layer "B.Cu") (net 18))
 (segment (start 148.35124 86.62924) (end 146.812 85.09) (width 0.25) (layer "B.Cu") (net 18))
 (segment (start 146.812 85.09) (end 146.812 71.108) (width 0.25) (layer "B.Cu") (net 18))
 (segment (start 148.336 88.138) (end 150.83028 88.138) (width 0.25) (layer "B.Cu") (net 19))
 (segment (start 150.83028 88.138) (end 151.50338 87.4649) (width 0.25) (layer "B.Cu") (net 19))
 (segment (start 145.542 70.104) (end 145.542 85.344) (width 0.25) (layer "B.Cu") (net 19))
 (segment (start 145.542 85.344) (end 148.336 88.138) (width 0.25) (layer "B.Cu") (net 19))
 (segment (start 172.72 60.829) (end 172.72 65.52) (width 0.25) (layer "B.Cu") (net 20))
 (segment (start 158.242 86.36) (end 156.464 88.138) (width 0.25) (layer "B.Cu") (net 20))
 (segment (start 153.96972 88.138) (end 153.29662 87.4649) (width 0.25) (layer "B.Cu") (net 20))
 (segment (start 169.406 68.834) (end 166.116 68.834) (width 0.25) (layer "B.Cu") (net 20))
 (segment (start 156.464 88.138) (end 153.96972 88.138) (width 0.25) (layer "B.Cu") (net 20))
 (segment (start 158.242 76.708) (end 158.242 86.36) (width 0.25) (layer "B.Cu") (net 20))
 (segment (start 172.72 65.52) (end 169.406 68.834) (width 0.25) (layer "B.Cu") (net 20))
 (segment (start 166.116 68.834) (end 158.242 76.708) (width 0.25) (layer "B.Cu") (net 20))
 (segment (start 157.48 60.829) (end 157.48 66.04) (width 0.25) (layer "B.Cu") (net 21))
 (segment (start 149.31136 74.20864) (end 149.31136 81.68894) (width 0.25) (layer "B.Cu") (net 21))
 (segment (start 157.48 66.04) (end 149.31136 74.20864) (width 0.25) (layer "B.Cu") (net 21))
 (segment (start 164.846 67.31) (end 165.85 67.31) (width 0.25) (layer "B.Cu") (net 22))
 (segment (start 167.64 65.52) (end 167.64 60.829) (width 0.25) (layer "B.Cu") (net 22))
 (segment (start 156.718 82.77606) (end 156.718 75.438) (width 0.25) (layer "B.Cu") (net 22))
 (segment (start 156.12618 83.36788) (end 156.718 82.77606) (width 0.25) (layer "B.Cu") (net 22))
 (segment (start 165.85 67.31) (end 167.64 65.52) (width 0.25) (layer "B.Cu") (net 22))
 (segment (start 156.718 75.438) (end 164.846 67.31) (width 0.25) (layer "B.Cu") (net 22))
 (segment (start 155.48864 75.39736) (end 155.48864 81.68894) (width 0.25) (layer "B.Cu") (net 23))
 (segment (start 165.1 64.139) (end 165.1 65.786) (width 0.25) (layer "B.Cu") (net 23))
 (segment (start 165.1 65.786) (end 155.48864 75.39736) (width 0.25) (layer "B.Cu") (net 23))
 (segment (start 167.132 74.168) (end 168.148 73.152) (width 0.25) (layer "B.Cu") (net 2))
 (segment (start 165.89756 75.40244) (end 167.132 74.168) (width 0.25) (layer "B.Cu") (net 2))
 (segment (start 168.148 73.152) (end 169.672 73.152) (width 0.25) (layer "B.Cu") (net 2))
 (segment (start 165.89756 80.49768) (end 165.89756 77.75956) (width 0.25) (layer "B.Cu") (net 2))
 (segment (start 165.89756 77.75956) (end 165.89756 75.40244) (width 0.25) (layer "B.Cu") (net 2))
 (segment (start 163.91382 83.36788) (end 163.068 82.52206) (width 0.25) (layer "B.Cu") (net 4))
 (segment (start 167.64 71.12) (end 168.91 71.12) (width 0.25) (layer "B.Cu") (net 4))
 (segment (start 163.068 75.946) (end 163.068 75.692) (width 0.25) (layer "B.Cu") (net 4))
 (segment (start 163.068 78.74) (end 163.068 75.946) (width 0.25) (layer "B.Cu") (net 4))
 (segment (start 163.068 75.692) (end 165.1 73.66) (width 0.25) (layer "B.Cu") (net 4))
 (segment (start 165.1 73.66) (end 167.64 71.12) (width 0.25) (layer "B.Cu") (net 4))
 (segment (start 163.068 82.52206) (end 163.068 78.74) (width 0.25) (layer "B.Cu") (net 4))
 (segment (start 162.306 85.344) (end 161.544 84.582) (width 0.25) (layer "B.Cu") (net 5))
 (segment (start 165.1508 86.62924) (end 163.59124 86.62924) (width 0.25) (layer "B.Cu") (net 5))
 (segment (start 163.59124 86.62924) (end 162.306 85.344) (width 0.25) (layer "B.Cu") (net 5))
 (segment (start 161.544 84.582) (end 161.544 81.534) (width 0.25) (layer "B.Cu") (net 5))
 (segment (start 166.37 69.85) (end 166.624 69.596) (width 0.25) (layer "B.Cu") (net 6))
 (segment (start 160.782 85.598) (end 160.782 83.312) (width 0.25) (layer "B.Cu") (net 6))
 (segment (start 163.217859 88.033859) (end 162.052 86.868) (width 0.25) (layer "B.Cu") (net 6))
 (segment (start 162.052 86.868) (end 160.782 85.598) (width 0.25) (layer "B.Cu") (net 6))
 (segment (start 166.174421 88.033859) (end 163.217859 88.033859) (width 0.25) (layer "B.Cu") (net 6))
 (segment (start 166.74338 87.4649) (end 166.174421 88.033859) (width 0.25) (layer "B.Cu") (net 6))
 (segment (start 160.782 75.438) (end 166.37 69.85) (width 0.25) (layer "B.Cu") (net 6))
 (segment (start 160.782 83.312) (end 160.782 75.438) (width 0.25) (layer "B.Cu") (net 6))
 (segment (start 166.624 69.596) (end 169.418 69.596) (width 0.25) (layer "B.Cu") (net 6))
 (segment (start 164.846 75.184) (end 168.148 71.882) (width 0.25) (layer "B.Cu") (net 8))
 (segment (start 164.55136 81.68894) (end 164.55136 78.52664) (width 0.25) (layer "B.Cu") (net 8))
 (segment (start 164.55136 75.47864) (end 164.846 75.184) (width 0.25) (layer "B.Cu") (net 8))
 (segment (start 164.55136 81.68894) (end 164.55136 75.47864) (width 0.25) (layer "B.Cu") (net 8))
 (segment (start 168.148 71.882) (end 169.164 71.882) (width 0.25) (layer "B.Cu") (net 8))
 (segment (start 166.37 71.12) (end 167.132 70.358) (width 0.25) (layer "B.Cu") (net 13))
 (segment (start 164.12972 85.15096) (end 163.63696 85.15096) (width 0.25) (layer "B.Cu") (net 13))
 (segment (start 162.306 75.184) (end 166.37 71.12) (width 0.25) (layer "B.Cu") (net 13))
 (segment (start 162.306 83.82) (end 162.306 78.994) (width 0.25) (layer "B.Cu") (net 13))
 (segment (start 167.132 70.358) (end 169.164 70.358) (width 0.25) (layer "B.Cu") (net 13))
 (segment (start 163.63696 85.15096) (end 162.306 83.82) (width 0.25) (layer "B.Cu") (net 13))
 (segment (start 162.306 78.994) (end 162.306 75.184) (width 0.25) (layer "B.Cu") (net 13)))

